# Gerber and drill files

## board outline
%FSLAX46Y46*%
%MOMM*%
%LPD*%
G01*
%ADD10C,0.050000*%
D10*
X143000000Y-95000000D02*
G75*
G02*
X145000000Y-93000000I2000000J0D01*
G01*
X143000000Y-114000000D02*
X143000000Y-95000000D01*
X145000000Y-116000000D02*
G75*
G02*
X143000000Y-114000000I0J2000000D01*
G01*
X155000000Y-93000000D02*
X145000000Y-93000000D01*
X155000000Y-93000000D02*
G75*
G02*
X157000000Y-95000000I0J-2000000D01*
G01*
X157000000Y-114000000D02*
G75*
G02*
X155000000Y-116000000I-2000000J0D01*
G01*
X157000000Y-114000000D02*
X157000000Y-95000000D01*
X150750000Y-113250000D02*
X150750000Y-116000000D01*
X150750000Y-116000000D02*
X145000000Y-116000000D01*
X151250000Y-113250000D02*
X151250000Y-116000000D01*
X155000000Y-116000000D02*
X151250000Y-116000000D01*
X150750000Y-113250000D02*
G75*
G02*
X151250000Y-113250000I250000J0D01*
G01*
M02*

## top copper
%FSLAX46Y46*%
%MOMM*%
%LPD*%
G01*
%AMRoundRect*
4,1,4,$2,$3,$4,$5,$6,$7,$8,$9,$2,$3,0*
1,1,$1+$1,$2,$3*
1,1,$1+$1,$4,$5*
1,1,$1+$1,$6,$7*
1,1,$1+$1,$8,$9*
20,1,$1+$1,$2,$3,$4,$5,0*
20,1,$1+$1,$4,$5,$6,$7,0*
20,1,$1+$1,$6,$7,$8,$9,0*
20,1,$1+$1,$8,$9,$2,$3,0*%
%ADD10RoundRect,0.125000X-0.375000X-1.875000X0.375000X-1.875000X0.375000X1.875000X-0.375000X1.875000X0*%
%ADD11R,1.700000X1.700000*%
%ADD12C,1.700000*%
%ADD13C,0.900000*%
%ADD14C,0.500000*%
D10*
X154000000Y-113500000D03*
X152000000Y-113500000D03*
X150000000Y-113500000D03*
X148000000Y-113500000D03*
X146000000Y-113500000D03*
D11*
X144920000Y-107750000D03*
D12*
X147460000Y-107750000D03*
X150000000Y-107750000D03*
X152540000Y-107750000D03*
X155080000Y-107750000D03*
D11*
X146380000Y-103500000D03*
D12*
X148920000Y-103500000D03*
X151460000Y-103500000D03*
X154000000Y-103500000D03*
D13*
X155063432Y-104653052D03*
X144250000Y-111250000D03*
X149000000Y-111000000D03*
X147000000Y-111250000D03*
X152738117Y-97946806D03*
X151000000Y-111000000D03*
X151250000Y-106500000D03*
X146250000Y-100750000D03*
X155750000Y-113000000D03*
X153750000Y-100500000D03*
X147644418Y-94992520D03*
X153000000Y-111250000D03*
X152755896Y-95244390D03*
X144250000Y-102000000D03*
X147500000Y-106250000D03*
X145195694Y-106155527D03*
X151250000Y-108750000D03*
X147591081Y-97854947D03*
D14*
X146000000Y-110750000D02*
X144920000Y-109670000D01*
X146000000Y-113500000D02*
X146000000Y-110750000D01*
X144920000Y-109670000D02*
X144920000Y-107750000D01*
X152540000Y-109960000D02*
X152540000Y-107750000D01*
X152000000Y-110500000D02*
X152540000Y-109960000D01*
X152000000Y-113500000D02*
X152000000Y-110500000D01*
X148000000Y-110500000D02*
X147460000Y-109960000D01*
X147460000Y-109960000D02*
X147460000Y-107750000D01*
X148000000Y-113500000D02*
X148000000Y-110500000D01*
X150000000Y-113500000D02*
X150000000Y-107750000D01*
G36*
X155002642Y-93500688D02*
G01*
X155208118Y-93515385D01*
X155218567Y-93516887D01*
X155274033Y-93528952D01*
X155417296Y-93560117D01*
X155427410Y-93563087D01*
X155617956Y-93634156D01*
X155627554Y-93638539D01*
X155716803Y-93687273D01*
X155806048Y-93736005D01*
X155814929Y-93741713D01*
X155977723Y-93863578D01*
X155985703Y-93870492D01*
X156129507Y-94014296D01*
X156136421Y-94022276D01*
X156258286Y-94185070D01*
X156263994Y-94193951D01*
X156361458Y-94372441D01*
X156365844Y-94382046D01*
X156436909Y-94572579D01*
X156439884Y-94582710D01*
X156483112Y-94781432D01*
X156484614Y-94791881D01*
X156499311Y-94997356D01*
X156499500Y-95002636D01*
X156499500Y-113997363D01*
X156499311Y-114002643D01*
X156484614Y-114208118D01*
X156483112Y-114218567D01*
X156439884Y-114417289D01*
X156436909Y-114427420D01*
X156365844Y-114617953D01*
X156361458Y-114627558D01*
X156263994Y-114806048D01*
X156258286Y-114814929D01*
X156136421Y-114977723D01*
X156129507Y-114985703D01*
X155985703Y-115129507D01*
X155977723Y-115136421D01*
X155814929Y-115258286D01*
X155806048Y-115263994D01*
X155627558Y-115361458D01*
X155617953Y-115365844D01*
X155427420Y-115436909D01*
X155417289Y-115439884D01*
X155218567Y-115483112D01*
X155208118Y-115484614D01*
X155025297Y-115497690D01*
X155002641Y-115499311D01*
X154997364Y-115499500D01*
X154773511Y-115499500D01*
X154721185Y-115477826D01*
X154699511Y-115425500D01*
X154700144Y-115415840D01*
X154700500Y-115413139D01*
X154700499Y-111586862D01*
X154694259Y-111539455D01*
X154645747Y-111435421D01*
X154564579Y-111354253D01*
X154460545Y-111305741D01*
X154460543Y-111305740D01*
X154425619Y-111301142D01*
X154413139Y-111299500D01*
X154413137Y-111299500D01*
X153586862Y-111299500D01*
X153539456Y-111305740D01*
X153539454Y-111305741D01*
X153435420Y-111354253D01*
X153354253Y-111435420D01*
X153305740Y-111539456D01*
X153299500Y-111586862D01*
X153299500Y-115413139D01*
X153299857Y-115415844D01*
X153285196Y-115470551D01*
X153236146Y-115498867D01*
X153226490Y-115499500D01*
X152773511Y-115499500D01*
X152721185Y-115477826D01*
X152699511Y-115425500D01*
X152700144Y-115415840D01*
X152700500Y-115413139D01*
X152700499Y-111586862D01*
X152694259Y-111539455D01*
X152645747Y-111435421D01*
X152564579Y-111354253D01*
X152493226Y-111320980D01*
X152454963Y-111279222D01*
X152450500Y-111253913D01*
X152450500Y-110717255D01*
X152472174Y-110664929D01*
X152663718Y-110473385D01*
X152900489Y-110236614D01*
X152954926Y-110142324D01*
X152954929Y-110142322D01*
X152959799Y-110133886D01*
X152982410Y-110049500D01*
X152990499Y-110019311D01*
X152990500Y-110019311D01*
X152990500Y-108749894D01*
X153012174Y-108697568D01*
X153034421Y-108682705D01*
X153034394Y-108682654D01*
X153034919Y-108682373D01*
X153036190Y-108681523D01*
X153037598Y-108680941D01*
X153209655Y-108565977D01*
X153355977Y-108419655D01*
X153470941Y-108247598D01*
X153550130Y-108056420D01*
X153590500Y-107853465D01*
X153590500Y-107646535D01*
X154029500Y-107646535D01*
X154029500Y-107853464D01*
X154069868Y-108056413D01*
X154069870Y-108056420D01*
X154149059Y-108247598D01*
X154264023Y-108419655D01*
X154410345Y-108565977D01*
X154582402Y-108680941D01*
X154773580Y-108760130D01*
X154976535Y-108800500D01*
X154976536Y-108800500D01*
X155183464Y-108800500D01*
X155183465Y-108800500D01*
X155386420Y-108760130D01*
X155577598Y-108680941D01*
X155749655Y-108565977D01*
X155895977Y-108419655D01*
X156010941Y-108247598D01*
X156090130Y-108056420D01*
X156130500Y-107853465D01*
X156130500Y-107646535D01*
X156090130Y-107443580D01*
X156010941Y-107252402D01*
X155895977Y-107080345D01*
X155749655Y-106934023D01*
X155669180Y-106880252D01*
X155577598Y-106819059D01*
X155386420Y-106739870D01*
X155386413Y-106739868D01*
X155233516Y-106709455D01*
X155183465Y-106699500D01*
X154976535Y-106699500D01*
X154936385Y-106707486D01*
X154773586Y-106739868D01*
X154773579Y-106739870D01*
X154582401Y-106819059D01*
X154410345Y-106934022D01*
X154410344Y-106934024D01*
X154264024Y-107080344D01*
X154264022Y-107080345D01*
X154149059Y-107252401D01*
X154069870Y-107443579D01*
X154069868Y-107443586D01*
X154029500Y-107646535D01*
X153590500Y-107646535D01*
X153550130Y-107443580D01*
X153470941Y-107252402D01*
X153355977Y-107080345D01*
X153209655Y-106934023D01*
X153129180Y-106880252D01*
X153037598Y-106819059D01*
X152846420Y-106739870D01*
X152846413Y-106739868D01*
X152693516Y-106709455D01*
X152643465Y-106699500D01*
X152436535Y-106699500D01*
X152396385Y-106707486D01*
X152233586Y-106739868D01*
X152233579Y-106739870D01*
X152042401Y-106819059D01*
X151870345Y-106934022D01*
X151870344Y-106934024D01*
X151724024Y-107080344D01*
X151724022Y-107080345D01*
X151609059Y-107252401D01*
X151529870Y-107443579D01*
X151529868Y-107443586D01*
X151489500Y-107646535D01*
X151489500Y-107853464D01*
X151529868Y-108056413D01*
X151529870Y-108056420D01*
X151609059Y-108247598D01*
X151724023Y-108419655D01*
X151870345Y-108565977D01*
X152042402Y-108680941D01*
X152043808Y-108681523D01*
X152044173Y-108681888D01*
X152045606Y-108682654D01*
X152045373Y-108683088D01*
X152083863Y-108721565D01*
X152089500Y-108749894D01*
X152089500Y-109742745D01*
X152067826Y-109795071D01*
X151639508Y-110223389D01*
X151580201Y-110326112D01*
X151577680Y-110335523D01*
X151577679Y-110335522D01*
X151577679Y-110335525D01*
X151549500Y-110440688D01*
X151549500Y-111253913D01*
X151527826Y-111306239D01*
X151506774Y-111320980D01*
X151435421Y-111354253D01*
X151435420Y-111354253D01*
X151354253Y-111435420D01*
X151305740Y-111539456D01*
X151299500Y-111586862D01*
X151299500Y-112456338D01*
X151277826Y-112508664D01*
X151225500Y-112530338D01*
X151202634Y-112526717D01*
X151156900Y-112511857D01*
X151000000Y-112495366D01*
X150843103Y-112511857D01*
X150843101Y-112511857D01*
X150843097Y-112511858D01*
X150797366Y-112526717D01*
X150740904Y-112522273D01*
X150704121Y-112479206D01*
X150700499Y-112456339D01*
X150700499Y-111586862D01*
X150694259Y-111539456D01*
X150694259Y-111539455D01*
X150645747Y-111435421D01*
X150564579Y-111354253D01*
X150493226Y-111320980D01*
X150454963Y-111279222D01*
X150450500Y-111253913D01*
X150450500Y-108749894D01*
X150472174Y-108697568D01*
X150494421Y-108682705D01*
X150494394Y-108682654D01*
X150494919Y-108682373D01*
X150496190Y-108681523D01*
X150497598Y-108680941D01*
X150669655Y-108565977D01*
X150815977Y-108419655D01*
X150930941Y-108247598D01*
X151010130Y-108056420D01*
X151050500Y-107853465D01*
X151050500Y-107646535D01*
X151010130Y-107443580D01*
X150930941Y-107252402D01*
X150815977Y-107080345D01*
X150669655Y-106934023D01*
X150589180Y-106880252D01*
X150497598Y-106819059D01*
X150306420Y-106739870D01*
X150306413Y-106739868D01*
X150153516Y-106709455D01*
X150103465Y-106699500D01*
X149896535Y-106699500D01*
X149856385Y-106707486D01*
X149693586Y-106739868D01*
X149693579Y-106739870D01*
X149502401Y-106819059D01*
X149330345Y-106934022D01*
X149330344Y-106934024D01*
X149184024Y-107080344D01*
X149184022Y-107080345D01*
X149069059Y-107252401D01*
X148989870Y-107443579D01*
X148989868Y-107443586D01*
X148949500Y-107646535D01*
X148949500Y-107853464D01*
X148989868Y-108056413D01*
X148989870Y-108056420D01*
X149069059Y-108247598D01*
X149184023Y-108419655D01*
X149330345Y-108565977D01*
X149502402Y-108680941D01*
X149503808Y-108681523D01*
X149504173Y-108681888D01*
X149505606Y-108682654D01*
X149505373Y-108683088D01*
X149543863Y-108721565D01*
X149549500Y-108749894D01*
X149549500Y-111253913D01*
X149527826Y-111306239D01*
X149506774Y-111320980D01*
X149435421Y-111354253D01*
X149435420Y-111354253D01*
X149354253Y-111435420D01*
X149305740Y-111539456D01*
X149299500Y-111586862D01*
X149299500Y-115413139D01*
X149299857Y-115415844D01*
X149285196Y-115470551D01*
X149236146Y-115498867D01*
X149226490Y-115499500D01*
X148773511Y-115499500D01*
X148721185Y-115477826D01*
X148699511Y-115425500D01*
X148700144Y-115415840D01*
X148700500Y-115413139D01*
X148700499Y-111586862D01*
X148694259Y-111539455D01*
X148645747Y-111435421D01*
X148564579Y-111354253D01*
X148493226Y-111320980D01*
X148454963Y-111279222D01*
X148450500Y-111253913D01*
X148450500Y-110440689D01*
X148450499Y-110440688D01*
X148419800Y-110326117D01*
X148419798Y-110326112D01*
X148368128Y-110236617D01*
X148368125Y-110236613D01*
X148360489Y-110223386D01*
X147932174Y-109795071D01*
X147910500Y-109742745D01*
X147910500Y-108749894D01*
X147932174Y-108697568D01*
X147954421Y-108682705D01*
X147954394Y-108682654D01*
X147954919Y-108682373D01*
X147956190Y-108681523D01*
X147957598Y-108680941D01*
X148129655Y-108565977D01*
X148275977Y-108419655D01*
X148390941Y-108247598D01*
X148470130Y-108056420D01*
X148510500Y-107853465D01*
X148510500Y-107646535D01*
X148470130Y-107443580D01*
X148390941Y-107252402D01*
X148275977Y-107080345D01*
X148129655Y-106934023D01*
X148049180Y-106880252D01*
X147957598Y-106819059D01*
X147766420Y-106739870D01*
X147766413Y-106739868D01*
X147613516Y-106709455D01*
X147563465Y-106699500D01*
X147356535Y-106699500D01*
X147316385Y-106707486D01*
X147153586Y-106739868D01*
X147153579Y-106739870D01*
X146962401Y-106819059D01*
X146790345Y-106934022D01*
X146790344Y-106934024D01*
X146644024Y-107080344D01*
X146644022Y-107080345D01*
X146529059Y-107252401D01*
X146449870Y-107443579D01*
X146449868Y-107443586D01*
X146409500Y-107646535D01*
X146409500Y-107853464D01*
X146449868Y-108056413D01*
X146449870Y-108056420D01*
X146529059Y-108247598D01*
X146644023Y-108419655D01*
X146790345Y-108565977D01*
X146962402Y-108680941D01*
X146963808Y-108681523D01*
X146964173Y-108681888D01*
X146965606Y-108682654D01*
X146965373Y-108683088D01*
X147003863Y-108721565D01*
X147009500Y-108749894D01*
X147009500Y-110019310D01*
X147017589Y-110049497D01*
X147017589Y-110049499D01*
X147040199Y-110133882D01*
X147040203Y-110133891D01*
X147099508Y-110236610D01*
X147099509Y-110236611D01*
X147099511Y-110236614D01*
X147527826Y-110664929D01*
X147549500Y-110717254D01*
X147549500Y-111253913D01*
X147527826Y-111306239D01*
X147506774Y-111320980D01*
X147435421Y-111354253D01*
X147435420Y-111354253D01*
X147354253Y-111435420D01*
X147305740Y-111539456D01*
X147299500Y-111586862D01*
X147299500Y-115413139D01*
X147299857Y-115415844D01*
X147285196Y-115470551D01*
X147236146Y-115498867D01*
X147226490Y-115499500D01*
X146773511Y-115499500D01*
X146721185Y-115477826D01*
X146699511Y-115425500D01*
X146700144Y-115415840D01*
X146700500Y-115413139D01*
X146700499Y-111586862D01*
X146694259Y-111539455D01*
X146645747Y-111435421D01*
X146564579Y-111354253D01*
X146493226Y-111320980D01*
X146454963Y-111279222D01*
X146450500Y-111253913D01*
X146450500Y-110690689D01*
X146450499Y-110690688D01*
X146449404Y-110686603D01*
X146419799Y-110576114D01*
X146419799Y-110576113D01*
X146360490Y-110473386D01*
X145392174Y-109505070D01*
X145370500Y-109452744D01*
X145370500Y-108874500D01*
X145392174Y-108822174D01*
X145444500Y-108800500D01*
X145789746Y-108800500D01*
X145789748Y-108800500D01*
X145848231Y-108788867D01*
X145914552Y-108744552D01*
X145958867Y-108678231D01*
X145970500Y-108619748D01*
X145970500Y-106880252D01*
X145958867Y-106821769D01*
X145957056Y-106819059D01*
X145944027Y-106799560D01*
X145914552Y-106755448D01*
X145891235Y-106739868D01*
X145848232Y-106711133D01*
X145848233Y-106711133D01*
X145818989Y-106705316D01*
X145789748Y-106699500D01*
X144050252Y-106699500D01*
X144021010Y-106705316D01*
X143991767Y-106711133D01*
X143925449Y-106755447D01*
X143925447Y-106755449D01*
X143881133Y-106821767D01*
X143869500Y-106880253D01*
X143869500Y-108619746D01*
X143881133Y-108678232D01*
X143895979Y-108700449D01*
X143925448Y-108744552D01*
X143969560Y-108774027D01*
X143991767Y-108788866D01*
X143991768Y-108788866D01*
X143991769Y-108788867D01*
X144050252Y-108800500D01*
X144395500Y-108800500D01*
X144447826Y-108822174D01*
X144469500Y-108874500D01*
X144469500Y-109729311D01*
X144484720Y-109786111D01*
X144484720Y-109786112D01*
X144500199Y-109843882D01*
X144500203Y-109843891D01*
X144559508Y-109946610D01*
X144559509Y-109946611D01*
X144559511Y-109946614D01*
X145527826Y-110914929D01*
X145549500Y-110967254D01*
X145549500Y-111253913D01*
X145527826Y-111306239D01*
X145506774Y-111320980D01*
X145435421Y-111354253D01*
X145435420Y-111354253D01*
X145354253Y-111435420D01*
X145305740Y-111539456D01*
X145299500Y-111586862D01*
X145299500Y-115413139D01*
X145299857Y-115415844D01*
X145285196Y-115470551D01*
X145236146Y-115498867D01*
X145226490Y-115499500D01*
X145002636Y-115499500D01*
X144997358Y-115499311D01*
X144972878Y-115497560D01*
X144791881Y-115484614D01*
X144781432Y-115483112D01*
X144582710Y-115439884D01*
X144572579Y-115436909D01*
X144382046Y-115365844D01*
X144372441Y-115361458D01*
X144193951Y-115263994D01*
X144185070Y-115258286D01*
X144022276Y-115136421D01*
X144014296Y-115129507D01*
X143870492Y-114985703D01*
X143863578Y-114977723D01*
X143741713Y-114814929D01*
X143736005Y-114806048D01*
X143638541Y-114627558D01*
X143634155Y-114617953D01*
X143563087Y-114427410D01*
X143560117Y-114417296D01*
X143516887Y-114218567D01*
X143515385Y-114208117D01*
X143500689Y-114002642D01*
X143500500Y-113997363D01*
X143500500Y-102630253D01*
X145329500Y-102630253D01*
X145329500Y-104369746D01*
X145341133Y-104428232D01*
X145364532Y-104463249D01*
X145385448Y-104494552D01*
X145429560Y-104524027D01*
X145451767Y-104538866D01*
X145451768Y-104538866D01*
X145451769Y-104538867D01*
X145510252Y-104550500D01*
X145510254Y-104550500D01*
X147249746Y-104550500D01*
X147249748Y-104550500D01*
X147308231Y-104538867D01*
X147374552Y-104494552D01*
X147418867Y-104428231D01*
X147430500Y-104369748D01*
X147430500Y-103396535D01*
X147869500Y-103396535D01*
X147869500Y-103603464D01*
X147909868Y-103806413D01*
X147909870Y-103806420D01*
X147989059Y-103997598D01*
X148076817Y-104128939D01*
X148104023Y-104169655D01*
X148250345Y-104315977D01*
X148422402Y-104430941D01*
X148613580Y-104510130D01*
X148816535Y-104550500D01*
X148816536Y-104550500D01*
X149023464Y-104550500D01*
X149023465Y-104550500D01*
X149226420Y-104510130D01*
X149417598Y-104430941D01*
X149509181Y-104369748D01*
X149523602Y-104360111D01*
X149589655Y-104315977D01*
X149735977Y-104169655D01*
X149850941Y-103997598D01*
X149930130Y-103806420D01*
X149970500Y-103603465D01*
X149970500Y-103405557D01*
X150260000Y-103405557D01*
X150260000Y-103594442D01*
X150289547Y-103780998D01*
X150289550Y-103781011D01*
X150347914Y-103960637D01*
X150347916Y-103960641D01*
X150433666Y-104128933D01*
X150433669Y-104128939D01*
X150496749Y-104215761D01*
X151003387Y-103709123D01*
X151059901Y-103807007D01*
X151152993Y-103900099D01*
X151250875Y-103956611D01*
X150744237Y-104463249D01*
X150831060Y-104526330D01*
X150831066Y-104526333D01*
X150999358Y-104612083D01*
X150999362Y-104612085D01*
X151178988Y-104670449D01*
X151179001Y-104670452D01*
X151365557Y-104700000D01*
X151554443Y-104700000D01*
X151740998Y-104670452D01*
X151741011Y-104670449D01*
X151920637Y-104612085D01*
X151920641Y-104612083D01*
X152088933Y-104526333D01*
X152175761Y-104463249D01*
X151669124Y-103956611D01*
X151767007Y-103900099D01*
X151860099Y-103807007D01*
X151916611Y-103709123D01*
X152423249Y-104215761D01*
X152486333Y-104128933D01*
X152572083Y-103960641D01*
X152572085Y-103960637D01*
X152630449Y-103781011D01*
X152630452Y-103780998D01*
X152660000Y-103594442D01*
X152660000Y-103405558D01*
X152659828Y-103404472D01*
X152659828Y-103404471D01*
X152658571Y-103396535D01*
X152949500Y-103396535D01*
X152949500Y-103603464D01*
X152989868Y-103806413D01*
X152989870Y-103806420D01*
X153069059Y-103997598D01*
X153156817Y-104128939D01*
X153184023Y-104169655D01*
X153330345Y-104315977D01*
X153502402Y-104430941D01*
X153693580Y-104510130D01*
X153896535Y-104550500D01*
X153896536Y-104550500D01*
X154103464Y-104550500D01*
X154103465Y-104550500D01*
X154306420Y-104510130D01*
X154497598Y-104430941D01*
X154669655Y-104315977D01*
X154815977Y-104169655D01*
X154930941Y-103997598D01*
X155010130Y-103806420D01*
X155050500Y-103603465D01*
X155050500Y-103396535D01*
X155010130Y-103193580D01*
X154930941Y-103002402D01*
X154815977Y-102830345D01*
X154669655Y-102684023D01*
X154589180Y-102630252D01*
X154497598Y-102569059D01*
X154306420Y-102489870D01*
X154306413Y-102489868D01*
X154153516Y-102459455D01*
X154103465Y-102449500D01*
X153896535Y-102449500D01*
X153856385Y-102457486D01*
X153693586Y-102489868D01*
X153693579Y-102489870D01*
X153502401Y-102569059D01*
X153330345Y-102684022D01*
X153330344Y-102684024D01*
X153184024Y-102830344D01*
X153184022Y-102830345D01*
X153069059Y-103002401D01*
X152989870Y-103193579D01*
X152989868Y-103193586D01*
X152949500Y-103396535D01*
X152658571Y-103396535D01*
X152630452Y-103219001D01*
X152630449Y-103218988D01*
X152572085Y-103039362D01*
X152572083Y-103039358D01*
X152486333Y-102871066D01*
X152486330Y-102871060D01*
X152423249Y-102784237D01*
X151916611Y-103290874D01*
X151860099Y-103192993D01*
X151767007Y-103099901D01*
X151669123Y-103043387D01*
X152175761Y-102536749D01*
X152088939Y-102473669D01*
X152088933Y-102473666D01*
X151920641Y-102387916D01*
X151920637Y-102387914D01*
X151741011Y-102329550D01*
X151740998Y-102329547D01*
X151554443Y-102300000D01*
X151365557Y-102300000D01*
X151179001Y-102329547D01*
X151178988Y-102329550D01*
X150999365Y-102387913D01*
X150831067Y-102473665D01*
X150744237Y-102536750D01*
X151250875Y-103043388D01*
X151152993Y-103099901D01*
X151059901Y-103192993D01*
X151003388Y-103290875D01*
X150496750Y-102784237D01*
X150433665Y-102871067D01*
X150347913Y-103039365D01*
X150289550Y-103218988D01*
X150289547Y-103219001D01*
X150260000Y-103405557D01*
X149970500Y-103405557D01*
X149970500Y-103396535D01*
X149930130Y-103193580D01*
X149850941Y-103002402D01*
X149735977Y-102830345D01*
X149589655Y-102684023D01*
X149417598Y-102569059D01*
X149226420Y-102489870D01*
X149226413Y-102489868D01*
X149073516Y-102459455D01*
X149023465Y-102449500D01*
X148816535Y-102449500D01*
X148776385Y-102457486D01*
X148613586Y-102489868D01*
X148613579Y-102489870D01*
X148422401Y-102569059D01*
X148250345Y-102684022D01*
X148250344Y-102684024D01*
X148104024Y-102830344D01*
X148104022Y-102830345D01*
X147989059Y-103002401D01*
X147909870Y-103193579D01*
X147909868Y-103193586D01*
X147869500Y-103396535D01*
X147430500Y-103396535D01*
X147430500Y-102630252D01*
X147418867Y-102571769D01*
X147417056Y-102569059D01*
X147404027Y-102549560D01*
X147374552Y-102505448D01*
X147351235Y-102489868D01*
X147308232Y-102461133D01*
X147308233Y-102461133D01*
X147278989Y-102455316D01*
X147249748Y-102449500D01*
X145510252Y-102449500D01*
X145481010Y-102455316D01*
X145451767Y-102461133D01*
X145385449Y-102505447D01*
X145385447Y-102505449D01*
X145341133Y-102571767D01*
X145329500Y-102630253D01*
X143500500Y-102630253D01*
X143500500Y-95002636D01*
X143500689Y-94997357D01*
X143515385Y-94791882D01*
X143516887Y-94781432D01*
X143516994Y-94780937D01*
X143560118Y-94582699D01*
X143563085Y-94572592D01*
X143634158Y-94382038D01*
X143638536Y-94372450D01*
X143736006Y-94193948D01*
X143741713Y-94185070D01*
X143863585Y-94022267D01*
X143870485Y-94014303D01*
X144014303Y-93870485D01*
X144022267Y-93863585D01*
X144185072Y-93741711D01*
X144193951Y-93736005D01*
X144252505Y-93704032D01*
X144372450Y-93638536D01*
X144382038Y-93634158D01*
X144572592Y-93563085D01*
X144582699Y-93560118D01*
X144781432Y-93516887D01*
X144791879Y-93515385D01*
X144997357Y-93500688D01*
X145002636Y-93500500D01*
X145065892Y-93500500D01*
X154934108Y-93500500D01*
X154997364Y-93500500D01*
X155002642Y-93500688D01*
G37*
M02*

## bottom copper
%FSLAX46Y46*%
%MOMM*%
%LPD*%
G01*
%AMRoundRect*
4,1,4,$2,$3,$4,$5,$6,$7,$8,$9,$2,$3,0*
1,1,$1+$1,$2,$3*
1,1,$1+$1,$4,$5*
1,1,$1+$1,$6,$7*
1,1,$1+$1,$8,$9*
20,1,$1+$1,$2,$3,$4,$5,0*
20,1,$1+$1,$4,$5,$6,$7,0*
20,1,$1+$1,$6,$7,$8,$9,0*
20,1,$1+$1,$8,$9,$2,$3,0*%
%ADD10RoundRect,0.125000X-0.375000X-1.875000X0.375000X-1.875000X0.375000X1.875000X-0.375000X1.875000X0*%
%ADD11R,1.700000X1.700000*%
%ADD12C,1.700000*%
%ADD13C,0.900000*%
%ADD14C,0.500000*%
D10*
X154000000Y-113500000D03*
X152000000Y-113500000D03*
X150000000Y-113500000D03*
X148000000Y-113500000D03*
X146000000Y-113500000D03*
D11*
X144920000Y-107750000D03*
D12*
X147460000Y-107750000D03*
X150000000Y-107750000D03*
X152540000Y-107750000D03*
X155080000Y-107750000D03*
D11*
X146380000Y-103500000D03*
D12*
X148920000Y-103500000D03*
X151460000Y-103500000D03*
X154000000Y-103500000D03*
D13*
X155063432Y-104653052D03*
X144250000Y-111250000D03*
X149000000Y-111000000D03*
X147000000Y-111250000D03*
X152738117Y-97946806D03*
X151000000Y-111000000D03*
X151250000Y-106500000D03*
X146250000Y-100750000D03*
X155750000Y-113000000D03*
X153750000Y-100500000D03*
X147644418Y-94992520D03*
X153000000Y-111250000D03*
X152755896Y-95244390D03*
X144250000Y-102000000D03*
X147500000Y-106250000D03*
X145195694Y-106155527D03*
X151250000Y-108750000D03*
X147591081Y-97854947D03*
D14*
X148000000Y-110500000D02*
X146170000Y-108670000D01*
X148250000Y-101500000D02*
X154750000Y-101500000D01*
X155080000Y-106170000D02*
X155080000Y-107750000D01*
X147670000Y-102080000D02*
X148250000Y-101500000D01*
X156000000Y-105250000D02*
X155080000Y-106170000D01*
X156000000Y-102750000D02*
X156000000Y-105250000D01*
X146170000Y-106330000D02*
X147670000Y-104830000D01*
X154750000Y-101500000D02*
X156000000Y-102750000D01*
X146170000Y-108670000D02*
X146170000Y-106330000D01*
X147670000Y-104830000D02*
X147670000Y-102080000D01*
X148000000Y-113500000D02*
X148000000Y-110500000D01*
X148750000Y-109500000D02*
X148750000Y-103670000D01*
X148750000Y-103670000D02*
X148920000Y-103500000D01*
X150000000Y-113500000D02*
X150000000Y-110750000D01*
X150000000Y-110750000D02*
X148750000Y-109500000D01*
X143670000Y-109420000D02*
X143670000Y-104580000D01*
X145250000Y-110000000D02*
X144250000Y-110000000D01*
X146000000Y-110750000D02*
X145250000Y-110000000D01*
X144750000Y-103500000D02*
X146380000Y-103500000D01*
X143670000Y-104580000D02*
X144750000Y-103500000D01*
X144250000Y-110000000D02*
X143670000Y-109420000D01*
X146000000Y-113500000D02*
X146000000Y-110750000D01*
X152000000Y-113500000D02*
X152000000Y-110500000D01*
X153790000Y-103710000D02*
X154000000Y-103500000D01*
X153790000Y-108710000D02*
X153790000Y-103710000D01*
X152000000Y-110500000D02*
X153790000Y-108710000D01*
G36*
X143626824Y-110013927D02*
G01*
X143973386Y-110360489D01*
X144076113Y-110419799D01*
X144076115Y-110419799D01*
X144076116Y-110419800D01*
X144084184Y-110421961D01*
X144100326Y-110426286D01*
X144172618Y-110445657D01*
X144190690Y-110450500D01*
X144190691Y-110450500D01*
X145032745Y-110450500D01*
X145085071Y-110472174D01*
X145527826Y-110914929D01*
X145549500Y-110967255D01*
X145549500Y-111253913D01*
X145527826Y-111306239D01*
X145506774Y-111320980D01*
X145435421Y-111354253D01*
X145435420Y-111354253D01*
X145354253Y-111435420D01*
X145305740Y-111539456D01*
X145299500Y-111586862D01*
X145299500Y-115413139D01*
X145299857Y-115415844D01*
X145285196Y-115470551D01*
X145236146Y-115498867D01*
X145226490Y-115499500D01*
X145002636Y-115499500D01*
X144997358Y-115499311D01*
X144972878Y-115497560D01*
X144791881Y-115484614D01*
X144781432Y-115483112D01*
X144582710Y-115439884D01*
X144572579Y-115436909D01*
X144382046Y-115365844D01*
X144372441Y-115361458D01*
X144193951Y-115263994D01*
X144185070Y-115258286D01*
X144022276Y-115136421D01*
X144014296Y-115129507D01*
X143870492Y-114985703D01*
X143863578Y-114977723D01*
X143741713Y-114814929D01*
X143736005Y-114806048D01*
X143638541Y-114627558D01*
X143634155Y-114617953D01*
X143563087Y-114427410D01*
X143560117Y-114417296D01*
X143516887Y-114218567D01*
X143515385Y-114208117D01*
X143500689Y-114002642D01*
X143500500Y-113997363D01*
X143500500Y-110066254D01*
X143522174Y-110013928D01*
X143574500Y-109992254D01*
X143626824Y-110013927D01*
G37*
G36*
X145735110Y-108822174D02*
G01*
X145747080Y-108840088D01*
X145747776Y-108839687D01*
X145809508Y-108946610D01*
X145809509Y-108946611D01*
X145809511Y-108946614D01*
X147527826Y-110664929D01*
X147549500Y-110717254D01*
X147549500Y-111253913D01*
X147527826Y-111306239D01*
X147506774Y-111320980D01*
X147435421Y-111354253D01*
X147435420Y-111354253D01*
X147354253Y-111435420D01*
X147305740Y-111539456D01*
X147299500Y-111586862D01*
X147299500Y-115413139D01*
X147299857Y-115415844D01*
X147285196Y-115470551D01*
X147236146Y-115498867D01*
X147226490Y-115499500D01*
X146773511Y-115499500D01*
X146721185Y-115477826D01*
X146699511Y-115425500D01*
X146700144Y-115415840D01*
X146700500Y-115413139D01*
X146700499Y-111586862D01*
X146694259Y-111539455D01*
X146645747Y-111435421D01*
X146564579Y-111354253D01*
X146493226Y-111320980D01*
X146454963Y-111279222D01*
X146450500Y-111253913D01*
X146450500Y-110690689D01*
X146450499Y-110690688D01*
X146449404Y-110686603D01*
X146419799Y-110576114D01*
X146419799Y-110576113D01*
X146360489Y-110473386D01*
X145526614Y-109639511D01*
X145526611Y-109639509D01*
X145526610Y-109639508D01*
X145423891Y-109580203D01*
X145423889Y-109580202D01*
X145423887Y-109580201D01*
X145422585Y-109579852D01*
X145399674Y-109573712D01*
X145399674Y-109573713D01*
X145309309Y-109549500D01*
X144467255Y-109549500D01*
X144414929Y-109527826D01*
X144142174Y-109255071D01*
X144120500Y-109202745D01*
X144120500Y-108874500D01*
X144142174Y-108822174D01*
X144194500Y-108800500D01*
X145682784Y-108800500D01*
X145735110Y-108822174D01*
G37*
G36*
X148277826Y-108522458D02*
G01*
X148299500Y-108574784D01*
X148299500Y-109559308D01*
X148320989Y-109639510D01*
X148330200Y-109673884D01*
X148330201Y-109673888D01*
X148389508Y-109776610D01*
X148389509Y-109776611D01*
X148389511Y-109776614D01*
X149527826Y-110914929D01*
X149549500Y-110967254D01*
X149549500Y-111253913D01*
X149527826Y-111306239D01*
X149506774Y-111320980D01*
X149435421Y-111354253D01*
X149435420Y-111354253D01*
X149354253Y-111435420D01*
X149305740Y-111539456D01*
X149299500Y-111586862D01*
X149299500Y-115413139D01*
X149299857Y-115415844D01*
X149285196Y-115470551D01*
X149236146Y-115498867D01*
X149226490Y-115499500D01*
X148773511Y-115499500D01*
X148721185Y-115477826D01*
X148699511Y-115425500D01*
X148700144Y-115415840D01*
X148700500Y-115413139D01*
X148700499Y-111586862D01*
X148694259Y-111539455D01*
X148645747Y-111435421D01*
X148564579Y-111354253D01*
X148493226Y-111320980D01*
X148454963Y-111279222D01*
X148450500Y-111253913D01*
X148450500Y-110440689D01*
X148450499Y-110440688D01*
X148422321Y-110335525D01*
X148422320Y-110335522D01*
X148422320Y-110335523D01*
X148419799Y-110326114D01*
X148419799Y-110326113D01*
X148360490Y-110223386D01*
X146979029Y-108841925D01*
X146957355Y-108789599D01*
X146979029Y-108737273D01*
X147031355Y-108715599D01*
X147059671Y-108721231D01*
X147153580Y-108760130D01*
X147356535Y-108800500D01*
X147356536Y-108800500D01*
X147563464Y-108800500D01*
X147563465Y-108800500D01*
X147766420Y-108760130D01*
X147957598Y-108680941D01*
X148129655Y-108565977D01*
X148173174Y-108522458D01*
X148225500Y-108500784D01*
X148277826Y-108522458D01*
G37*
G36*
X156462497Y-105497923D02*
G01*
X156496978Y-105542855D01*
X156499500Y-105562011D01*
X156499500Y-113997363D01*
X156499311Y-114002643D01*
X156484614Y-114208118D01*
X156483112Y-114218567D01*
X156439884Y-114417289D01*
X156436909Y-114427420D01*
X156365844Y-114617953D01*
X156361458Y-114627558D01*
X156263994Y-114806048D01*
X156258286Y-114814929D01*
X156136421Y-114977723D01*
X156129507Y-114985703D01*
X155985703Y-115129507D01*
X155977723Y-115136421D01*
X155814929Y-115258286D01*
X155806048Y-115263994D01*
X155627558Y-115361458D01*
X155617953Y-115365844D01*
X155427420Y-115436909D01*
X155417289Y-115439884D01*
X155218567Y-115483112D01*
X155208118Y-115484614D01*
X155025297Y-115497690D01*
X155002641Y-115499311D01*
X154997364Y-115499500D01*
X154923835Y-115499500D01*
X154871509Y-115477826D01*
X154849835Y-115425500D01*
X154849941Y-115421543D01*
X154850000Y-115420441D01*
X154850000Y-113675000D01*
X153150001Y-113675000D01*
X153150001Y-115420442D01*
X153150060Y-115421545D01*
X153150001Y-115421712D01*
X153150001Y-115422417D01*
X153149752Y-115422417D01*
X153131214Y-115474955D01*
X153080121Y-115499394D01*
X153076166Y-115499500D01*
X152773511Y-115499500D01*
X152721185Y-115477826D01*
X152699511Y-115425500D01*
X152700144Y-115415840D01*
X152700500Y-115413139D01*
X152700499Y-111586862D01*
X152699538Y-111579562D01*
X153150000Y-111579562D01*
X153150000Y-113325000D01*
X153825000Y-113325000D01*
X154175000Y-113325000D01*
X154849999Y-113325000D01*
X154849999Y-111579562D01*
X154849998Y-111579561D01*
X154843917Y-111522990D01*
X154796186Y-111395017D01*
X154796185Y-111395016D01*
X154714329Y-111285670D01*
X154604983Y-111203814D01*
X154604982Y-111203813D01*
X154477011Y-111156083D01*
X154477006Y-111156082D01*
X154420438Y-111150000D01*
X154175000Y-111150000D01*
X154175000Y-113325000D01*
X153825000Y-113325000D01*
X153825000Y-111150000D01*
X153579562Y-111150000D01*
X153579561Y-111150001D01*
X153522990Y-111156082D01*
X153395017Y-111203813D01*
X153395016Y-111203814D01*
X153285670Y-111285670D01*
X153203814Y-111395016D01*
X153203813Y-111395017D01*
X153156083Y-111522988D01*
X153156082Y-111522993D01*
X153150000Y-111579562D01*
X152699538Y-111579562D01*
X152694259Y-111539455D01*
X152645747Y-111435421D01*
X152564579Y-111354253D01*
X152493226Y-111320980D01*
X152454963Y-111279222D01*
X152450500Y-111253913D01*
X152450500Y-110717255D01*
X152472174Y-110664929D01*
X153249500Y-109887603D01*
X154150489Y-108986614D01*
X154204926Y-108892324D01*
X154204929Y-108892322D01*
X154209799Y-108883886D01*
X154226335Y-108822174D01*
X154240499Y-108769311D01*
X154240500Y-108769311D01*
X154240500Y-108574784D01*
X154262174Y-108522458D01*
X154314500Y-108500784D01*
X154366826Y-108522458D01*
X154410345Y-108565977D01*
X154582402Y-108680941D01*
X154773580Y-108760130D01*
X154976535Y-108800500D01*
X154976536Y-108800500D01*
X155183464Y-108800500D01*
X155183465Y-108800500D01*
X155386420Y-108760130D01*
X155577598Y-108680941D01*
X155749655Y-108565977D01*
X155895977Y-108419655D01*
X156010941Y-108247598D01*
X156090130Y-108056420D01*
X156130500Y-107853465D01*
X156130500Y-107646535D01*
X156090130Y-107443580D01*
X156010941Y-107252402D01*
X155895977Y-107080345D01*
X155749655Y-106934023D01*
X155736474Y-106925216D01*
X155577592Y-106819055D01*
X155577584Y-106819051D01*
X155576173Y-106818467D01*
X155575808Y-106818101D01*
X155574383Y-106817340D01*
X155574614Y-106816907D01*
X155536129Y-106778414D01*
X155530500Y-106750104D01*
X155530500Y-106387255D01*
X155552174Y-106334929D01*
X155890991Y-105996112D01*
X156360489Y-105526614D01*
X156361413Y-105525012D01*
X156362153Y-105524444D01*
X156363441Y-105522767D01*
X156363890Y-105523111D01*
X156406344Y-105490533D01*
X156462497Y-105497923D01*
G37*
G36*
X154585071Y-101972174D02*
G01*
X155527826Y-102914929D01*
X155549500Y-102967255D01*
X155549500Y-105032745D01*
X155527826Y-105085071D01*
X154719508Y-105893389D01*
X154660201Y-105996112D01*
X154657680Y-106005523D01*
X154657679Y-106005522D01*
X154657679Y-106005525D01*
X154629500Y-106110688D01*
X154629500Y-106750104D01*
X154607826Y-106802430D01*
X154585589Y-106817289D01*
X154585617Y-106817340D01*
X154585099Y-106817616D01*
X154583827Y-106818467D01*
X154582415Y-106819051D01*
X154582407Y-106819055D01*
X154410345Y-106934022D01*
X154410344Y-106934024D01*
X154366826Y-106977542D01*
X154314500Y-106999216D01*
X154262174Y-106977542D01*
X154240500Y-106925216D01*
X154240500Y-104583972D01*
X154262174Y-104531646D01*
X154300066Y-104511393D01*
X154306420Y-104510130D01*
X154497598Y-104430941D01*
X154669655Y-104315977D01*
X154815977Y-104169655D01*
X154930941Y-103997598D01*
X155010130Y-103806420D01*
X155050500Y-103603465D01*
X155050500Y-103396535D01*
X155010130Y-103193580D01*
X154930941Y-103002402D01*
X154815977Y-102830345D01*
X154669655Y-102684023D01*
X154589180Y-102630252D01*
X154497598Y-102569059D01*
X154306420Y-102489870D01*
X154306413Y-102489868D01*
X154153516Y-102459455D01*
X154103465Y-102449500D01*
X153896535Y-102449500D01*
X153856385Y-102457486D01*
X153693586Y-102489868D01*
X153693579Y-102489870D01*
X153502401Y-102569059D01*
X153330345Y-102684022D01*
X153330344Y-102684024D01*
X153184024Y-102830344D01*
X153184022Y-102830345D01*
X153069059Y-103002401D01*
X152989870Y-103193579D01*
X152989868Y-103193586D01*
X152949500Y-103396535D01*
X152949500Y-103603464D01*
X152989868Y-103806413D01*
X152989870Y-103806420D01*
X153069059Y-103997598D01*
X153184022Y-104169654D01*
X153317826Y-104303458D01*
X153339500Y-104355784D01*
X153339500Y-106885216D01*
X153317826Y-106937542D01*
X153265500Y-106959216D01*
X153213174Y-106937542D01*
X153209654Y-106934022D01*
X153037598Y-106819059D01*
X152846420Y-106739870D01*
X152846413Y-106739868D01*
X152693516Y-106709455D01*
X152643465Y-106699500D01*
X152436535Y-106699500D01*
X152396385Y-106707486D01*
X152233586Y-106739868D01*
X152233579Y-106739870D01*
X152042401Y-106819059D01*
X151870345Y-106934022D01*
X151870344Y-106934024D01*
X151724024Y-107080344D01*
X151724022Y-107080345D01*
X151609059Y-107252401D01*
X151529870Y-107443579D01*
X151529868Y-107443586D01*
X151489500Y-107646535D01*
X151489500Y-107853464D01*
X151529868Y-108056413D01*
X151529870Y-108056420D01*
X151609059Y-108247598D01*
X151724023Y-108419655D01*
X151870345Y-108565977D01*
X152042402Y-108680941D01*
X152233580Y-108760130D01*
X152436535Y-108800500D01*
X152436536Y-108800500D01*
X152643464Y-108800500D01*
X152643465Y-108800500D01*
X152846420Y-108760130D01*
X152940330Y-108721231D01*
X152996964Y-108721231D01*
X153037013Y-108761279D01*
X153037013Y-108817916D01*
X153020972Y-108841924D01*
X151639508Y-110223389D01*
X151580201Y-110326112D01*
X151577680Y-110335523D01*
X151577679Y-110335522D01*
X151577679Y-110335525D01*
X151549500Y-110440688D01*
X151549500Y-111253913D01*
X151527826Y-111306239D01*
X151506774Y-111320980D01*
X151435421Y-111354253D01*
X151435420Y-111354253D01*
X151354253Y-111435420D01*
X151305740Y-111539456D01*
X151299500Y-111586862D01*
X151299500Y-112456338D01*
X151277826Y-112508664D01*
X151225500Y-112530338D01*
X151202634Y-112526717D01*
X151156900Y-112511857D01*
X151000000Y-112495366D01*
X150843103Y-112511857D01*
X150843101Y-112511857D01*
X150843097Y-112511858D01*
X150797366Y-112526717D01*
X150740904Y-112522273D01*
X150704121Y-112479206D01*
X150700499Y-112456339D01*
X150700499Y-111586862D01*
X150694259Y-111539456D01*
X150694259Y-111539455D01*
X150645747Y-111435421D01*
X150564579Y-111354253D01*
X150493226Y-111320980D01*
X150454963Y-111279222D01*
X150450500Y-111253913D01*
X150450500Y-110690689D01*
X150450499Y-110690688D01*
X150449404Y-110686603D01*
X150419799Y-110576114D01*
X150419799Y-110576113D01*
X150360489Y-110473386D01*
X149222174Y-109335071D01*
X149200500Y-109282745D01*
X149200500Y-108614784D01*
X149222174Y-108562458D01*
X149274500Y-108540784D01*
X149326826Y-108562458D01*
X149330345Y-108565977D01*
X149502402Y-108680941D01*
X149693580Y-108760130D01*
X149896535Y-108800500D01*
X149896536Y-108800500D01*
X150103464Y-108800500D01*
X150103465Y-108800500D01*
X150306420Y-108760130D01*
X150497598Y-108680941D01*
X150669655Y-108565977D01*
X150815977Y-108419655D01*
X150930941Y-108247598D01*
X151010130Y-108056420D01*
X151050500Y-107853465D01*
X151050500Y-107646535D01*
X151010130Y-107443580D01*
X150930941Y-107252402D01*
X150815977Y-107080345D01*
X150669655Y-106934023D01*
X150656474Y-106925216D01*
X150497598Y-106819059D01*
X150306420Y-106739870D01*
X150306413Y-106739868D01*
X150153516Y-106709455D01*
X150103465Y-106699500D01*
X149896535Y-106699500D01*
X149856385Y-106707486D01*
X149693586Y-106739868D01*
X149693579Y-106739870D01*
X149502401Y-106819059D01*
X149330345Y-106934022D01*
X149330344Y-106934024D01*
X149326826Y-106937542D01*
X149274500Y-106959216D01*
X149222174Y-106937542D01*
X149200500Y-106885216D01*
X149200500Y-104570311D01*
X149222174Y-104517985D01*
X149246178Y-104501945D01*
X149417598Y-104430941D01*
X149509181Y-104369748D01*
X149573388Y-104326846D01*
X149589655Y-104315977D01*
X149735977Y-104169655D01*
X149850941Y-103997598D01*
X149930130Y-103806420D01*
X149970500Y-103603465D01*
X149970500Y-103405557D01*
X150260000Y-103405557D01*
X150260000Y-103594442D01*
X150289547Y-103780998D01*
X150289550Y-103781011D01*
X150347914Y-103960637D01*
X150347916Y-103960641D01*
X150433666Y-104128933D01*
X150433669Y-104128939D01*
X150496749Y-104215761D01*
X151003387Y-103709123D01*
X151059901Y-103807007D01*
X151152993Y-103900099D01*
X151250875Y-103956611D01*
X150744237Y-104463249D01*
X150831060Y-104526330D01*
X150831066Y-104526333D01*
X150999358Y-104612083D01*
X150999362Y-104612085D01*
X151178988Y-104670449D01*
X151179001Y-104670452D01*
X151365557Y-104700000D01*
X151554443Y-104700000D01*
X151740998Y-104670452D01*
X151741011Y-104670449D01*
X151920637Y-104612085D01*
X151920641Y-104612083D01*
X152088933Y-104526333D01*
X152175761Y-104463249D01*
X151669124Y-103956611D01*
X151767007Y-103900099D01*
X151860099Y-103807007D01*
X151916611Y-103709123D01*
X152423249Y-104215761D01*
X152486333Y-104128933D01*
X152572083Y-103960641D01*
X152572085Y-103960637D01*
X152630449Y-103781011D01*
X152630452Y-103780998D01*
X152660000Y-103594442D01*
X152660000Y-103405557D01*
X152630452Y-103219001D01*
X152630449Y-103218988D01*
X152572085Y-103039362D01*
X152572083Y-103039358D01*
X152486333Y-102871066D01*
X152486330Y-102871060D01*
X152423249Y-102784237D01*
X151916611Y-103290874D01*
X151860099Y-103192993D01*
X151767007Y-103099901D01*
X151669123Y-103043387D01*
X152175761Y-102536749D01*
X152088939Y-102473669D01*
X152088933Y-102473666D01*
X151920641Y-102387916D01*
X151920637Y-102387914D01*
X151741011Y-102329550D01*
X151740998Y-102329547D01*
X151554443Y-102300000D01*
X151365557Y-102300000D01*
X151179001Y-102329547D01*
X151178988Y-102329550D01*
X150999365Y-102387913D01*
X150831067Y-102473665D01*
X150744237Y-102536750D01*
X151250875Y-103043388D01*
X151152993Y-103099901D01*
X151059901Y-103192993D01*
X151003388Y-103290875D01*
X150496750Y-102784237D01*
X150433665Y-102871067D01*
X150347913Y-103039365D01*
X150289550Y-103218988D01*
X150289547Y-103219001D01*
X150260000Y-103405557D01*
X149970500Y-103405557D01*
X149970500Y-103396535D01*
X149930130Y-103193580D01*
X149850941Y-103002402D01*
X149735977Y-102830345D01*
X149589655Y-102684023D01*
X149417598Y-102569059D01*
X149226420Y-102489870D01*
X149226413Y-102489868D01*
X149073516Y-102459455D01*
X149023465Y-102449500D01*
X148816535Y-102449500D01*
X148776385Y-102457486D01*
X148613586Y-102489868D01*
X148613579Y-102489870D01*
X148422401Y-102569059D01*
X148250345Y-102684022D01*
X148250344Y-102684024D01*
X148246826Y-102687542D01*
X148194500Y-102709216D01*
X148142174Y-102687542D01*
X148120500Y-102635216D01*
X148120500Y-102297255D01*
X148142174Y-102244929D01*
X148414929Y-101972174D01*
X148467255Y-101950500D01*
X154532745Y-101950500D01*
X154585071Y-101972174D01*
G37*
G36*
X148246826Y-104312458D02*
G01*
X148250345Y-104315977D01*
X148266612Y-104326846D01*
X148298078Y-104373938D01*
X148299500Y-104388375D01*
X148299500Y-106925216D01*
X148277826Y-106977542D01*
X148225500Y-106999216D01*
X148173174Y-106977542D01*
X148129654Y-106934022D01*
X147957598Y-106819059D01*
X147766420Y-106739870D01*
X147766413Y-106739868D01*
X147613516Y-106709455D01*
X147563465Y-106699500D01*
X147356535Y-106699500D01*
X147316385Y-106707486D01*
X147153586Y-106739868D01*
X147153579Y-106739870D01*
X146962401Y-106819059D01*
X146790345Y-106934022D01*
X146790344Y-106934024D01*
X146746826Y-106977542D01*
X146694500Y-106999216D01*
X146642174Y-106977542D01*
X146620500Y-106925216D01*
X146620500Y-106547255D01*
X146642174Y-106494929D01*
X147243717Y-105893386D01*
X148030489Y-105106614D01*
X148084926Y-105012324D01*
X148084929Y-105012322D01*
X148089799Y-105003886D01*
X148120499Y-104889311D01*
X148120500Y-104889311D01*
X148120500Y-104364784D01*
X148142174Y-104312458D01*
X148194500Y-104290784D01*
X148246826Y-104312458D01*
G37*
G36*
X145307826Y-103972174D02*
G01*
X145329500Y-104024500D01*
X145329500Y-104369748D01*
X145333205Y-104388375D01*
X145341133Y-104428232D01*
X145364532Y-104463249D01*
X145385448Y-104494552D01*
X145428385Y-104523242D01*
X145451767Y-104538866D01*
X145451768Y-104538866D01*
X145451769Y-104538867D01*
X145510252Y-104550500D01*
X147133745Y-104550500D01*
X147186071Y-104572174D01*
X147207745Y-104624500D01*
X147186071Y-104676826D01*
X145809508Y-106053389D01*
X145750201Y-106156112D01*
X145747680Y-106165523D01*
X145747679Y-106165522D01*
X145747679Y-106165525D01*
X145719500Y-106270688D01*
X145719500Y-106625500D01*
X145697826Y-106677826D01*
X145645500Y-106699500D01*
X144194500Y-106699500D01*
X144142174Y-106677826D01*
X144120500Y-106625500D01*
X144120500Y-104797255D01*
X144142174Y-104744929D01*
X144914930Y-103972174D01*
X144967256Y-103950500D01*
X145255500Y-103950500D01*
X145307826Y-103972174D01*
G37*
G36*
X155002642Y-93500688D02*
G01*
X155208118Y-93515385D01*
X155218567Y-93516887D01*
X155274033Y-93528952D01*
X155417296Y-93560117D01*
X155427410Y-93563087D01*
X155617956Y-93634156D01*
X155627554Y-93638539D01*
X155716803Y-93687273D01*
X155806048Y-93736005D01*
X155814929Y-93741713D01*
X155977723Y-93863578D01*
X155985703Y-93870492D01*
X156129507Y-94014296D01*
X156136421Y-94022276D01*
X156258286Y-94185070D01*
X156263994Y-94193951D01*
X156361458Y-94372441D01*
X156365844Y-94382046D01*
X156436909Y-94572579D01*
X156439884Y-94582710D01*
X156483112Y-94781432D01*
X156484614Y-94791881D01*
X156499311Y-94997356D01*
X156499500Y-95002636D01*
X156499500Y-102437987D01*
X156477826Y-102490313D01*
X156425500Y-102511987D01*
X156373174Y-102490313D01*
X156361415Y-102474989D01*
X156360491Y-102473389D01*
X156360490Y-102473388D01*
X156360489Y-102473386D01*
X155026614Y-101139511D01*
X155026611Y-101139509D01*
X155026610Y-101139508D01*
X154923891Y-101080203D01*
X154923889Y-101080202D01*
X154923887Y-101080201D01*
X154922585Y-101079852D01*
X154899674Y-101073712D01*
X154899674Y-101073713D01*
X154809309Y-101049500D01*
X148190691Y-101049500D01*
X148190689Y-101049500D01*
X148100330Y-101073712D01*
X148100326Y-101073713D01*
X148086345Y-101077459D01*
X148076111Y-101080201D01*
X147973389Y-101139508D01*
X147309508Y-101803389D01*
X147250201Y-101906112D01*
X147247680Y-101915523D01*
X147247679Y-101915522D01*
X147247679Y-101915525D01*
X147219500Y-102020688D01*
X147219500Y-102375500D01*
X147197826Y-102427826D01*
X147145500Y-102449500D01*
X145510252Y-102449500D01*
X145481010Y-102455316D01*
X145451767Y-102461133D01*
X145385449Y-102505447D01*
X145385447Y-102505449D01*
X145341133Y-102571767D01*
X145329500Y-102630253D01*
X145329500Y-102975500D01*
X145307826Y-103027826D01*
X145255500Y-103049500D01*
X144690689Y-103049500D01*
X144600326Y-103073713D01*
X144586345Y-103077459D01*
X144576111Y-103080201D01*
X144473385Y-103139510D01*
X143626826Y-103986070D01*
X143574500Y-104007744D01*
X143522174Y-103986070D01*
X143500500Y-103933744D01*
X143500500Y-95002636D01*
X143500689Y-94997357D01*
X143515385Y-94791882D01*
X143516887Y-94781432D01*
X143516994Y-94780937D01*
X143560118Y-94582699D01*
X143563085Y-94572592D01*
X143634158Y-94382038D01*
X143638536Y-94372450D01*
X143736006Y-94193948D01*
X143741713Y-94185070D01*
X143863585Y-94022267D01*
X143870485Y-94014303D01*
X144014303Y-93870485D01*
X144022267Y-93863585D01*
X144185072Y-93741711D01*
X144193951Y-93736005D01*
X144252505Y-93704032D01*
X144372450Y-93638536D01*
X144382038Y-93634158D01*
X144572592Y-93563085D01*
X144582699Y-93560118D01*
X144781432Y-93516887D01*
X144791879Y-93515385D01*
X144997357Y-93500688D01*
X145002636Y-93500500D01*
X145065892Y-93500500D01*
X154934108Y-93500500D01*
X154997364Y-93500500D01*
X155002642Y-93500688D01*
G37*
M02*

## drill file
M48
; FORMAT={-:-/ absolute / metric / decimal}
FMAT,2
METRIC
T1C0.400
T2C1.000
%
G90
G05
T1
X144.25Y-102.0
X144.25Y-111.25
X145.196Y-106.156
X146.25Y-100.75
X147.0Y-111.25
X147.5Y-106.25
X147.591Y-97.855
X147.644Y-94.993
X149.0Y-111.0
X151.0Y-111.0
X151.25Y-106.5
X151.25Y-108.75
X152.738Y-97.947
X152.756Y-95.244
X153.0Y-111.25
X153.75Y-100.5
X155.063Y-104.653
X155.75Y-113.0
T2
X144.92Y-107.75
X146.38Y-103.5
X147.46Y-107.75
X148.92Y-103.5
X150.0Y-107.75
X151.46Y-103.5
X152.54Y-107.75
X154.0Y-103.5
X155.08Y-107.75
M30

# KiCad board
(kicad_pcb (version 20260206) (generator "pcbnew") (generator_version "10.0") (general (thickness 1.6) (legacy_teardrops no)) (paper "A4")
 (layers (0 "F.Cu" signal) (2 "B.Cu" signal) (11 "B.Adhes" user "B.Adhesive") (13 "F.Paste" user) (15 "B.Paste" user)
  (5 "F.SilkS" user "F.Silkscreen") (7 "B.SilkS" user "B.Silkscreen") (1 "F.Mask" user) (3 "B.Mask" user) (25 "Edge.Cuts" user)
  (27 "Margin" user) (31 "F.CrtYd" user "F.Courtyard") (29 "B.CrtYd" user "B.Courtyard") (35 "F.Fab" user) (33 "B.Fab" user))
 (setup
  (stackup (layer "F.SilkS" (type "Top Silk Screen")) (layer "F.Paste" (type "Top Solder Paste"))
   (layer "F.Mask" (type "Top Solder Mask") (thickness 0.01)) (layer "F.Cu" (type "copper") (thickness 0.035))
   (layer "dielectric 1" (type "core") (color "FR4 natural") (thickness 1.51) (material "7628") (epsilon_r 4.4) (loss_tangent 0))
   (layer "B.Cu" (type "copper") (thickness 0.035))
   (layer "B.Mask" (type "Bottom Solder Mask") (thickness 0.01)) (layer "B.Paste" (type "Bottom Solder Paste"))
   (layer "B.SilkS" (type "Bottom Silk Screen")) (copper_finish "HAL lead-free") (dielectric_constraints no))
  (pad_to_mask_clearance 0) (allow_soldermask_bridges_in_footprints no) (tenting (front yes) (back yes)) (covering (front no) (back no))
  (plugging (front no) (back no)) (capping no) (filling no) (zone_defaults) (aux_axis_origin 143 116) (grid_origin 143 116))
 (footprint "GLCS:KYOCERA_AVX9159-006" (layer "F.Cu") (at 147 116 180)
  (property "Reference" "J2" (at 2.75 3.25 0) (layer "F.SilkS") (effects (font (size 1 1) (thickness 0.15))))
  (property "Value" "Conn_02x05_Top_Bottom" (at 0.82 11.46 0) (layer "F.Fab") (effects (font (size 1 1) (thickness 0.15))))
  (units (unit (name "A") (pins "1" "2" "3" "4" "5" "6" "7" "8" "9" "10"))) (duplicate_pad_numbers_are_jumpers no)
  (fp_line (start -3.75 2.75) (end -3.75 0) (stroke (width 0.05) (type default)) (layer "Edge.Cuts"))
  (fp_line (start -3.75 0) (end 2 0) (stroke (width 0.05) (type default)) (layer "Edge.Cuts"))
  (fp_line (start -4.25 2.75) (end -4.25 0) (stroke (width 0.05) (type default)) (layer "Edge.Cuts"))
  (fp_line (start -8 0) (end -4.25 0) (stroke (width 0.05) (type default)) (layer "Edge.Cuts"))
  (fp_arc (start -3.75 2.75) (mid -4 3) (end -4.25 2.75) (stroke (width 0.05) (type default)) (layer "Edge.Cuts"))
  (pad "1" smd roundrect (at -7 2.5) (size 1 4) (layers "F.Cu" "F.Mask" "F.Paste") (roundrect_rratio 0.125)
   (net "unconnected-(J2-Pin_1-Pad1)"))
  (pad "2" smd roundrect (at -5 2.5) (size 1 4) (layers "F.Cu" "F.Mask" "F.Paste") (roundrect_rratio 0.125) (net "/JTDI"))
  (pad "3" smd roundrect (at -3 2.5) (size 1 4) (layers "F.Cu" "F.Mask" "F.Paste") (roundrect_rratio 0.125) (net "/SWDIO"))
  (pad "4" smd roundrect (at -1 2.5) (size 1 4) (layers "F.Cu" "F.Mask" "F.Paste") (roundrect_rratio 0.125) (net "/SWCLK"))
  (pad "5" smd roundrect (at 1 2.5) (size 1 4) (layers "F.Cu" "F.Mask" "F.Paste") (roundrect_rratio 0.125) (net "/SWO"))
  (pad "6" smd roundrect (at -7 2.5) (size 1 4) (layers "B.Cu" "B.Mask" "B.Paste") (roundrect_rratio 0.125) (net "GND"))
  (pad "7" smd roundrect (at -5 2.5) (size 1 4) (layers "B.Cu" "B.Mask" "B.Paste") (roundrect_rratio 0.125) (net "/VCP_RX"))
  (pad "8" smd roundrect (at -3 2.5) (size 1 4) (layers "B.Cu" "B.Mask" "B.Paste") (roundrect_rratio 0.125) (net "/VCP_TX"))
  (pad "9" smd roundrect (at -1 2.5) (size 1 4) (layers "B.Cu" "B.Mask" "B.Paste") (roundrect_rratio 0.125) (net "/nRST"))
  (pad "10" smd roundrect (at 1 2.5) (size 1 4) (layers "B.Cu" "B.Mask" "B.Paste") (roundrect_rratio 0.125) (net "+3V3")))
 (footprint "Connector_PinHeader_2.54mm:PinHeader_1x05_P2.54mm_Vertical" (layer "F.Cu") (at 144.92 107.75 90)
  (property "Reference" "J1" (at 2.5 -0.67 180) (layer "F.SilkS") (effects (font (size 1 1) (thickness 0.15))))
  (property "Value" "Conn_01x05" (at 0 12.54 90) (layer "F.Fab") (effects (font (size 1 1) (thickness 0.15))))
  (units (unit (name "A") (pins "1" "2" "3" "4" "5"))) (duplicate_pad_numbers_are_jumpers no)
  (pad "1" thru_hole rect (at 0 0 90) (size 1.7 1.7) (drill 1) (layers "*.Cu" "*.Mask") (remove_unused_layers no) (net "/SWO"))
  (pad "2" thru_hole circle (at 0 2.54 90) (size 1.7 1.7) (drill 1) (layers "*.Cu" "*.Mask") (remove_unused_layers no) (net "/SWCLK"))
  (pad "3" thru_hole circle (at 0 5.08 90) (size 1.7 1.7) (drill 1) (layers "*.Cu" "*.Mask") (remove_unused_layers no) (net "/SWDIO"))
  (pad "4" thru_hole circle (at 0 7.62 90) (size 1.7 1.7) (drill 1) (layers "*.Cu" "*.Mask") (remove_unused_layers no) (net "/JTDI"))
  (pad "5" thru_hole circle (at 0 10.16 90) (size 1.7 1.7) (drill 1) (layers "*.Cu" "*.Mask") (remove_unused_layers no) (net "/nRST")))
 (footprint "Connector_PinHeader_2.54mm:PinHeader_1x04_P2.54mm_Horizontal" (layer "F.Cu") (at 146.38 103.5 90)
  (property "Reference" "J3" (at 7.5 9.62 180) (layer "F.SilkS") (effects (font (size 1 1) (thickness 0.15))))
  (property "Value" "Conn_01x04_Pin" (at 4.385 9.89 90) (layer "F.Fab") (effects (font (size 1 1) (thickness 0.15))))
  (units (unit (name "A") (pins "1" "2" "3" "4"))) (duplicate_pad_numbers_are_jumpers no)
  (pad "1" thru_hole rect (at 0 0 90) (size 1.7 1.7) (drill 1) (layers "*.Cu" "*.Mask") (remove_unused_layers no) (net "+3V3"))
  (pad "2" thru_hole circle (at 0 2.54 90) (size 1.7 1.7) (drill 1) (layers "*.Cu" "*.Mask") (remove_unused_layers no) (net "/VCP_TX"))
  (pad "3" thru_hole circle (at 0 5.08 90) (size 1.7 1.7) (drill 1) (layers "*.Cu" "*.Mask") (remove_unused_layers no) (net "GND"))
  (pad "4" thru_hole circle (at 0 7.62 90) (size 1.7 1.7) (drill 1) (layers "*.Cu" "*.Mask") (remove_unused_layers no) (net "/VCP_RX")))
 (gr_arc (start 143 95) (mid 143.585786 93.585786) (end 145 93) (stroke (width 0.05) (type default)) (layer "Edge.Cuts"))
 (gr_line (start 143 114) (end 143 95) (stroke (width 0.05) (type default)) (layer "Edge.Cuts"))
 (gr_arc (start 145 116) (mid 143.585786 115.414214) (end 143 114) (stroke (width 0.05) (type default)) (layer "Edge.Cuts"))
 (gr_line (start 155 93) (end 145 93) (stroke (width 0.05) (type default)) (layer "Edge.Cuts"))
 (gr_arc (start 155 93) (mid 156.414214 93.585786) (end 157 95) (stroke (width 0.05) (type default)) (layer "Edge.Cuts"))
 (gr_arc (start 157 114) (mid 156.414214 115.414214) (end 155 116) (stroke (width 0.05) (type default)) (layer "Edge.Cuts"))
 (gr_line (start 157 114) (end 157 95) (stroke (width 0.05) (type default)) (layer "Edge.Cuts"))
 (segment (start 146 110.75) (end 144.92 109.67) (width 0.5) (layer "F.Cu") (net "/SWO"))
 (segment (start 146 113.5) (end 146 110.75) (width 0.5) (layer "F.Cu") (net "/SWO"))
 (segment (start 144.92 109.67) (end 144.92 107.75) (width 0.5) (layer "F.Cu") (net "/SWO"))
 (segment (start 152.54 109.96) (end 152.54 107.75) (width 0.5) (layer "F.Cu") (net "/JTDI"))
 (segment (start 152 110.5) (end 152.54 109.96) (width 0.5) (layer "F.Cu") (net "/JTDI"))
 (segment (start 152 113.5) (end 152 110.5) (width 0.5) (layer "F.Cu") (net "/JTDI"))
 (segment (start 148 110.5) (end 146.17 108.67) (width 0.5) (layer "B.Cu") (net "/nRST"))
 (segment (start 148.25 101.5) (end 154.75 101.5) (width 0.5) (layer "B.Cu") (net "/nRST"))
 (segment (start 155.08 106.17) (end 155.08 107.75) (width 0.5) (layer "B.Cu") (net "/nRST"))
 (segment (start 147.67 102.08) (end 148.25 101.5) (width 0.5) (layer "B.Cu") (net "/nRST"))
 (segment (start 156 105.25) (end 155.08 106.17) (width 0.5) (layer "B.Cu") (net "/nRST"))
 (segment (start 156 102.75) (end 156 105.25) (width 0.5) (layer "B.Cu") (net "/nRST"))
 (segment (start 146.17 106.33) (end 147.67 104.83) (width 0.5) (layer "B.Cu") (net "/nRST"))
 (segment (start 154.75 101.5) (end 156 102.75) (width 0.5) (layer "B.Cu") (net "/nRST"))
 (segment (start 146.17 108.67) (end 146.17 106.33) (width 0.5) (layer "B.Cu") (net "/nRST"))
 (segment (start 147.67 104.83) (end 147.67 102.08) (width 0.5) (layer "B.Cu") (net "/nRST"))
 (segment (start 148 113.5) (end 148 110.5) (width 0.5) (layer "B.Cu") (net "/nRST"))
 (segment (start 148 110.5) (end 147.46 109.96) (width 0.5) (layer "F.Cu") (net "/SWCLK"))
 (segment (start 147.46 109.96) (end 147.46 107.75) (width 0.5) (layer "F.Cu") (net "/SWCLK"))
 (segment (start 148 113.5) (end 148 110.5) (width 0.5) (layer "F.Cu") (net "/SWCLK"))
 (segment (start 150 113.5) (end 150 107.75) (width 0.5) (layer "F.Cu") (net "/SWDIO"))
 (segment (start 148.75 109.5) (end 148.75 103.67) (width 0.5) (layer "B.Cu") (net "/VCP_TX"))
 (segment (start 148.75 103.67) (end 148.92 103.5) (width 0.5) (layer "B.Cu") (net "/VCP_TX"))
 (segment (start 150 113.5) (end 150 110.75) (width 0.5) (layer "B.Cu") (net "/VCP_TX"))
 (segment (start 150 110.75) (end 148.75 109.5) (width 0.5) (layer "B.Cu") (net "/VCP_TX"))
 (segment (start 143.67 109.42) (end 143.67 104.58) (width 0.5) (layer "B.Cu") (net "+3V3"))
 (segment (start 145.25 110) (end 144.25 110) (width 0.5) (layer "B.Cu") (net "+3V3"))
 (segment (start 146 110.75) (end 145.25 110) (width 0.5) (layer "B.Cu") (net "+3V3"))
 (segment (start 144.75 103.5) (end 146.38 103.5) (width 0.5) (layer "B.Cu") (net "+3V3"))
 (segment (start 143.67 104.58) (end 144.75 103.5) (width 0.5) (layer "B.Cu") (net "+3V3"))
 (segment (start 144.25 110) (end 143.67 109.42) (width 0.5) (layer "B.Cu") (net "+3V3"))
 (segment (start 146 113.5) (end 146 110.75) (width 0.5) (layer "B.Cu") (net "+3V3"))
 (segment (start 152 113.5) (end 152 110.5) (width 0.5) (layer "B.Cu") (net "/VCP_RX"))
 (segment (start 153.79 103.71) (end 154 103.5) (width 0.5) (layer "B.Cu") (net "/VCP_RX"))
 (segment (start 153.79 108.71) (end 153.79 103.71) (width 0.5) (layer "B.Cu") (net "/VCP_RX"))
 (segment (start 152 110.5) (end 153.79 108.71) (width 0.5) (layer "B.Cu") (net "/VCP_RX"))
 (via (at 155.063432 104.653052) (size 0.9) (drill 0.4) (layers "F.Cu" "B.Cu") (free yes) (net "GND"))
 (via (at 144.25 111.25) (size 0.9) (drill 0.4) (layers "F.Cu" "B.Cu") (free yes) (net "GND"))
 (via (at 149 111) (size 0.9) (drill 0.4) (layers "F.Cu" "B.Cu") (free yes) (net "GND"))
 (via (at 147 111.25) (size 0.9) (drill 0.4) (layers "F.Cu" "B.Cu") (free yes) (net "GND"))
 (via (at 152.738117 97.946806) (size 0.9) (drill 0.4) (layers "F.Cu" "B.Cu") (free yes) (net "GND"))
 (via (at 151 111) (size 0.9) (drill 0.4) (layers "F.Cu" "B.Cu") (free yes) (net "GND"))
 (via (at 151.25 106.5) (size 0.9) (drill 0.4) (layers "F.Cu" "B.Cu") (free yes) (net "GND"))
 (via (at 146.25 100.75) (size 0.9) (drill 0.4) (layers "F.Cu" "B.Cu") (free yes) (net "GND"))
 (via (at 155.75 113) (size 0.9) (drill 0.4) (layers "F.Cu" "B.Cu") (free yes) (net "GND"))
 (via (at 153.75 100.5) (size 0.9) (drill 0.4) (layers "F.Cu" "B.Cu") (free yes) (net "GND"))
 (via (at 147.644418 94.99252) (size 0.9) (drill 0.4) (layers "F.Cu" "B.Cu") (free yes) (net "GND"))
 (via (at 153 111.25) (size 0.9) (drill 0.4) (layers "F.Cu" "B.Cu") (free yes) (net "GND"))
 (via (at 152.755896 95.24439) (size 0.9) (drill 0.4) (layers "F.Cu" "B.Cu") (free yes) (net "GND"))
 (via (at 144.25 102) (size 0.9) (drill 0.4) (layers "F.Cu" "B.Cu") (free yes) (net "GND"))
 (via (at 147.5 106.25) (size 0.9) (drill 0.4) (layers "F.Cu" "B.Cu") (free yes) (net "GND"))
 (via (at 145.195694 106.155527) (size 0.9) (drill 0.4) (layers "F.Cu" "B.Cu") (free yes) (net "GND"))
 (via (at 151.25 108.75) (size 0.9) (drill 0.4) (layers "F.Cu" "B.Cu") (free yes) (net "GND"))
 (via (at 147.591081 97.854947) (size 0.9) (drill 0.4) (layers "F.Cu" "B.Cu") (free yes) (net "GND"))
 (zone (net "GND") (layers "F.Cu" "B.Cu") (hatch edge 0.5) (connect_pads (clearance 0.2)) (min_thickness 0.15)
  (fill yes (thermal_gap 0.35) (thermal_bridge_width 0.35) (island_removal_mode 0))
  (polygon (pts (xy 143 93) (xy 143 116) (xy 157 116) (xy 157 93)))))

